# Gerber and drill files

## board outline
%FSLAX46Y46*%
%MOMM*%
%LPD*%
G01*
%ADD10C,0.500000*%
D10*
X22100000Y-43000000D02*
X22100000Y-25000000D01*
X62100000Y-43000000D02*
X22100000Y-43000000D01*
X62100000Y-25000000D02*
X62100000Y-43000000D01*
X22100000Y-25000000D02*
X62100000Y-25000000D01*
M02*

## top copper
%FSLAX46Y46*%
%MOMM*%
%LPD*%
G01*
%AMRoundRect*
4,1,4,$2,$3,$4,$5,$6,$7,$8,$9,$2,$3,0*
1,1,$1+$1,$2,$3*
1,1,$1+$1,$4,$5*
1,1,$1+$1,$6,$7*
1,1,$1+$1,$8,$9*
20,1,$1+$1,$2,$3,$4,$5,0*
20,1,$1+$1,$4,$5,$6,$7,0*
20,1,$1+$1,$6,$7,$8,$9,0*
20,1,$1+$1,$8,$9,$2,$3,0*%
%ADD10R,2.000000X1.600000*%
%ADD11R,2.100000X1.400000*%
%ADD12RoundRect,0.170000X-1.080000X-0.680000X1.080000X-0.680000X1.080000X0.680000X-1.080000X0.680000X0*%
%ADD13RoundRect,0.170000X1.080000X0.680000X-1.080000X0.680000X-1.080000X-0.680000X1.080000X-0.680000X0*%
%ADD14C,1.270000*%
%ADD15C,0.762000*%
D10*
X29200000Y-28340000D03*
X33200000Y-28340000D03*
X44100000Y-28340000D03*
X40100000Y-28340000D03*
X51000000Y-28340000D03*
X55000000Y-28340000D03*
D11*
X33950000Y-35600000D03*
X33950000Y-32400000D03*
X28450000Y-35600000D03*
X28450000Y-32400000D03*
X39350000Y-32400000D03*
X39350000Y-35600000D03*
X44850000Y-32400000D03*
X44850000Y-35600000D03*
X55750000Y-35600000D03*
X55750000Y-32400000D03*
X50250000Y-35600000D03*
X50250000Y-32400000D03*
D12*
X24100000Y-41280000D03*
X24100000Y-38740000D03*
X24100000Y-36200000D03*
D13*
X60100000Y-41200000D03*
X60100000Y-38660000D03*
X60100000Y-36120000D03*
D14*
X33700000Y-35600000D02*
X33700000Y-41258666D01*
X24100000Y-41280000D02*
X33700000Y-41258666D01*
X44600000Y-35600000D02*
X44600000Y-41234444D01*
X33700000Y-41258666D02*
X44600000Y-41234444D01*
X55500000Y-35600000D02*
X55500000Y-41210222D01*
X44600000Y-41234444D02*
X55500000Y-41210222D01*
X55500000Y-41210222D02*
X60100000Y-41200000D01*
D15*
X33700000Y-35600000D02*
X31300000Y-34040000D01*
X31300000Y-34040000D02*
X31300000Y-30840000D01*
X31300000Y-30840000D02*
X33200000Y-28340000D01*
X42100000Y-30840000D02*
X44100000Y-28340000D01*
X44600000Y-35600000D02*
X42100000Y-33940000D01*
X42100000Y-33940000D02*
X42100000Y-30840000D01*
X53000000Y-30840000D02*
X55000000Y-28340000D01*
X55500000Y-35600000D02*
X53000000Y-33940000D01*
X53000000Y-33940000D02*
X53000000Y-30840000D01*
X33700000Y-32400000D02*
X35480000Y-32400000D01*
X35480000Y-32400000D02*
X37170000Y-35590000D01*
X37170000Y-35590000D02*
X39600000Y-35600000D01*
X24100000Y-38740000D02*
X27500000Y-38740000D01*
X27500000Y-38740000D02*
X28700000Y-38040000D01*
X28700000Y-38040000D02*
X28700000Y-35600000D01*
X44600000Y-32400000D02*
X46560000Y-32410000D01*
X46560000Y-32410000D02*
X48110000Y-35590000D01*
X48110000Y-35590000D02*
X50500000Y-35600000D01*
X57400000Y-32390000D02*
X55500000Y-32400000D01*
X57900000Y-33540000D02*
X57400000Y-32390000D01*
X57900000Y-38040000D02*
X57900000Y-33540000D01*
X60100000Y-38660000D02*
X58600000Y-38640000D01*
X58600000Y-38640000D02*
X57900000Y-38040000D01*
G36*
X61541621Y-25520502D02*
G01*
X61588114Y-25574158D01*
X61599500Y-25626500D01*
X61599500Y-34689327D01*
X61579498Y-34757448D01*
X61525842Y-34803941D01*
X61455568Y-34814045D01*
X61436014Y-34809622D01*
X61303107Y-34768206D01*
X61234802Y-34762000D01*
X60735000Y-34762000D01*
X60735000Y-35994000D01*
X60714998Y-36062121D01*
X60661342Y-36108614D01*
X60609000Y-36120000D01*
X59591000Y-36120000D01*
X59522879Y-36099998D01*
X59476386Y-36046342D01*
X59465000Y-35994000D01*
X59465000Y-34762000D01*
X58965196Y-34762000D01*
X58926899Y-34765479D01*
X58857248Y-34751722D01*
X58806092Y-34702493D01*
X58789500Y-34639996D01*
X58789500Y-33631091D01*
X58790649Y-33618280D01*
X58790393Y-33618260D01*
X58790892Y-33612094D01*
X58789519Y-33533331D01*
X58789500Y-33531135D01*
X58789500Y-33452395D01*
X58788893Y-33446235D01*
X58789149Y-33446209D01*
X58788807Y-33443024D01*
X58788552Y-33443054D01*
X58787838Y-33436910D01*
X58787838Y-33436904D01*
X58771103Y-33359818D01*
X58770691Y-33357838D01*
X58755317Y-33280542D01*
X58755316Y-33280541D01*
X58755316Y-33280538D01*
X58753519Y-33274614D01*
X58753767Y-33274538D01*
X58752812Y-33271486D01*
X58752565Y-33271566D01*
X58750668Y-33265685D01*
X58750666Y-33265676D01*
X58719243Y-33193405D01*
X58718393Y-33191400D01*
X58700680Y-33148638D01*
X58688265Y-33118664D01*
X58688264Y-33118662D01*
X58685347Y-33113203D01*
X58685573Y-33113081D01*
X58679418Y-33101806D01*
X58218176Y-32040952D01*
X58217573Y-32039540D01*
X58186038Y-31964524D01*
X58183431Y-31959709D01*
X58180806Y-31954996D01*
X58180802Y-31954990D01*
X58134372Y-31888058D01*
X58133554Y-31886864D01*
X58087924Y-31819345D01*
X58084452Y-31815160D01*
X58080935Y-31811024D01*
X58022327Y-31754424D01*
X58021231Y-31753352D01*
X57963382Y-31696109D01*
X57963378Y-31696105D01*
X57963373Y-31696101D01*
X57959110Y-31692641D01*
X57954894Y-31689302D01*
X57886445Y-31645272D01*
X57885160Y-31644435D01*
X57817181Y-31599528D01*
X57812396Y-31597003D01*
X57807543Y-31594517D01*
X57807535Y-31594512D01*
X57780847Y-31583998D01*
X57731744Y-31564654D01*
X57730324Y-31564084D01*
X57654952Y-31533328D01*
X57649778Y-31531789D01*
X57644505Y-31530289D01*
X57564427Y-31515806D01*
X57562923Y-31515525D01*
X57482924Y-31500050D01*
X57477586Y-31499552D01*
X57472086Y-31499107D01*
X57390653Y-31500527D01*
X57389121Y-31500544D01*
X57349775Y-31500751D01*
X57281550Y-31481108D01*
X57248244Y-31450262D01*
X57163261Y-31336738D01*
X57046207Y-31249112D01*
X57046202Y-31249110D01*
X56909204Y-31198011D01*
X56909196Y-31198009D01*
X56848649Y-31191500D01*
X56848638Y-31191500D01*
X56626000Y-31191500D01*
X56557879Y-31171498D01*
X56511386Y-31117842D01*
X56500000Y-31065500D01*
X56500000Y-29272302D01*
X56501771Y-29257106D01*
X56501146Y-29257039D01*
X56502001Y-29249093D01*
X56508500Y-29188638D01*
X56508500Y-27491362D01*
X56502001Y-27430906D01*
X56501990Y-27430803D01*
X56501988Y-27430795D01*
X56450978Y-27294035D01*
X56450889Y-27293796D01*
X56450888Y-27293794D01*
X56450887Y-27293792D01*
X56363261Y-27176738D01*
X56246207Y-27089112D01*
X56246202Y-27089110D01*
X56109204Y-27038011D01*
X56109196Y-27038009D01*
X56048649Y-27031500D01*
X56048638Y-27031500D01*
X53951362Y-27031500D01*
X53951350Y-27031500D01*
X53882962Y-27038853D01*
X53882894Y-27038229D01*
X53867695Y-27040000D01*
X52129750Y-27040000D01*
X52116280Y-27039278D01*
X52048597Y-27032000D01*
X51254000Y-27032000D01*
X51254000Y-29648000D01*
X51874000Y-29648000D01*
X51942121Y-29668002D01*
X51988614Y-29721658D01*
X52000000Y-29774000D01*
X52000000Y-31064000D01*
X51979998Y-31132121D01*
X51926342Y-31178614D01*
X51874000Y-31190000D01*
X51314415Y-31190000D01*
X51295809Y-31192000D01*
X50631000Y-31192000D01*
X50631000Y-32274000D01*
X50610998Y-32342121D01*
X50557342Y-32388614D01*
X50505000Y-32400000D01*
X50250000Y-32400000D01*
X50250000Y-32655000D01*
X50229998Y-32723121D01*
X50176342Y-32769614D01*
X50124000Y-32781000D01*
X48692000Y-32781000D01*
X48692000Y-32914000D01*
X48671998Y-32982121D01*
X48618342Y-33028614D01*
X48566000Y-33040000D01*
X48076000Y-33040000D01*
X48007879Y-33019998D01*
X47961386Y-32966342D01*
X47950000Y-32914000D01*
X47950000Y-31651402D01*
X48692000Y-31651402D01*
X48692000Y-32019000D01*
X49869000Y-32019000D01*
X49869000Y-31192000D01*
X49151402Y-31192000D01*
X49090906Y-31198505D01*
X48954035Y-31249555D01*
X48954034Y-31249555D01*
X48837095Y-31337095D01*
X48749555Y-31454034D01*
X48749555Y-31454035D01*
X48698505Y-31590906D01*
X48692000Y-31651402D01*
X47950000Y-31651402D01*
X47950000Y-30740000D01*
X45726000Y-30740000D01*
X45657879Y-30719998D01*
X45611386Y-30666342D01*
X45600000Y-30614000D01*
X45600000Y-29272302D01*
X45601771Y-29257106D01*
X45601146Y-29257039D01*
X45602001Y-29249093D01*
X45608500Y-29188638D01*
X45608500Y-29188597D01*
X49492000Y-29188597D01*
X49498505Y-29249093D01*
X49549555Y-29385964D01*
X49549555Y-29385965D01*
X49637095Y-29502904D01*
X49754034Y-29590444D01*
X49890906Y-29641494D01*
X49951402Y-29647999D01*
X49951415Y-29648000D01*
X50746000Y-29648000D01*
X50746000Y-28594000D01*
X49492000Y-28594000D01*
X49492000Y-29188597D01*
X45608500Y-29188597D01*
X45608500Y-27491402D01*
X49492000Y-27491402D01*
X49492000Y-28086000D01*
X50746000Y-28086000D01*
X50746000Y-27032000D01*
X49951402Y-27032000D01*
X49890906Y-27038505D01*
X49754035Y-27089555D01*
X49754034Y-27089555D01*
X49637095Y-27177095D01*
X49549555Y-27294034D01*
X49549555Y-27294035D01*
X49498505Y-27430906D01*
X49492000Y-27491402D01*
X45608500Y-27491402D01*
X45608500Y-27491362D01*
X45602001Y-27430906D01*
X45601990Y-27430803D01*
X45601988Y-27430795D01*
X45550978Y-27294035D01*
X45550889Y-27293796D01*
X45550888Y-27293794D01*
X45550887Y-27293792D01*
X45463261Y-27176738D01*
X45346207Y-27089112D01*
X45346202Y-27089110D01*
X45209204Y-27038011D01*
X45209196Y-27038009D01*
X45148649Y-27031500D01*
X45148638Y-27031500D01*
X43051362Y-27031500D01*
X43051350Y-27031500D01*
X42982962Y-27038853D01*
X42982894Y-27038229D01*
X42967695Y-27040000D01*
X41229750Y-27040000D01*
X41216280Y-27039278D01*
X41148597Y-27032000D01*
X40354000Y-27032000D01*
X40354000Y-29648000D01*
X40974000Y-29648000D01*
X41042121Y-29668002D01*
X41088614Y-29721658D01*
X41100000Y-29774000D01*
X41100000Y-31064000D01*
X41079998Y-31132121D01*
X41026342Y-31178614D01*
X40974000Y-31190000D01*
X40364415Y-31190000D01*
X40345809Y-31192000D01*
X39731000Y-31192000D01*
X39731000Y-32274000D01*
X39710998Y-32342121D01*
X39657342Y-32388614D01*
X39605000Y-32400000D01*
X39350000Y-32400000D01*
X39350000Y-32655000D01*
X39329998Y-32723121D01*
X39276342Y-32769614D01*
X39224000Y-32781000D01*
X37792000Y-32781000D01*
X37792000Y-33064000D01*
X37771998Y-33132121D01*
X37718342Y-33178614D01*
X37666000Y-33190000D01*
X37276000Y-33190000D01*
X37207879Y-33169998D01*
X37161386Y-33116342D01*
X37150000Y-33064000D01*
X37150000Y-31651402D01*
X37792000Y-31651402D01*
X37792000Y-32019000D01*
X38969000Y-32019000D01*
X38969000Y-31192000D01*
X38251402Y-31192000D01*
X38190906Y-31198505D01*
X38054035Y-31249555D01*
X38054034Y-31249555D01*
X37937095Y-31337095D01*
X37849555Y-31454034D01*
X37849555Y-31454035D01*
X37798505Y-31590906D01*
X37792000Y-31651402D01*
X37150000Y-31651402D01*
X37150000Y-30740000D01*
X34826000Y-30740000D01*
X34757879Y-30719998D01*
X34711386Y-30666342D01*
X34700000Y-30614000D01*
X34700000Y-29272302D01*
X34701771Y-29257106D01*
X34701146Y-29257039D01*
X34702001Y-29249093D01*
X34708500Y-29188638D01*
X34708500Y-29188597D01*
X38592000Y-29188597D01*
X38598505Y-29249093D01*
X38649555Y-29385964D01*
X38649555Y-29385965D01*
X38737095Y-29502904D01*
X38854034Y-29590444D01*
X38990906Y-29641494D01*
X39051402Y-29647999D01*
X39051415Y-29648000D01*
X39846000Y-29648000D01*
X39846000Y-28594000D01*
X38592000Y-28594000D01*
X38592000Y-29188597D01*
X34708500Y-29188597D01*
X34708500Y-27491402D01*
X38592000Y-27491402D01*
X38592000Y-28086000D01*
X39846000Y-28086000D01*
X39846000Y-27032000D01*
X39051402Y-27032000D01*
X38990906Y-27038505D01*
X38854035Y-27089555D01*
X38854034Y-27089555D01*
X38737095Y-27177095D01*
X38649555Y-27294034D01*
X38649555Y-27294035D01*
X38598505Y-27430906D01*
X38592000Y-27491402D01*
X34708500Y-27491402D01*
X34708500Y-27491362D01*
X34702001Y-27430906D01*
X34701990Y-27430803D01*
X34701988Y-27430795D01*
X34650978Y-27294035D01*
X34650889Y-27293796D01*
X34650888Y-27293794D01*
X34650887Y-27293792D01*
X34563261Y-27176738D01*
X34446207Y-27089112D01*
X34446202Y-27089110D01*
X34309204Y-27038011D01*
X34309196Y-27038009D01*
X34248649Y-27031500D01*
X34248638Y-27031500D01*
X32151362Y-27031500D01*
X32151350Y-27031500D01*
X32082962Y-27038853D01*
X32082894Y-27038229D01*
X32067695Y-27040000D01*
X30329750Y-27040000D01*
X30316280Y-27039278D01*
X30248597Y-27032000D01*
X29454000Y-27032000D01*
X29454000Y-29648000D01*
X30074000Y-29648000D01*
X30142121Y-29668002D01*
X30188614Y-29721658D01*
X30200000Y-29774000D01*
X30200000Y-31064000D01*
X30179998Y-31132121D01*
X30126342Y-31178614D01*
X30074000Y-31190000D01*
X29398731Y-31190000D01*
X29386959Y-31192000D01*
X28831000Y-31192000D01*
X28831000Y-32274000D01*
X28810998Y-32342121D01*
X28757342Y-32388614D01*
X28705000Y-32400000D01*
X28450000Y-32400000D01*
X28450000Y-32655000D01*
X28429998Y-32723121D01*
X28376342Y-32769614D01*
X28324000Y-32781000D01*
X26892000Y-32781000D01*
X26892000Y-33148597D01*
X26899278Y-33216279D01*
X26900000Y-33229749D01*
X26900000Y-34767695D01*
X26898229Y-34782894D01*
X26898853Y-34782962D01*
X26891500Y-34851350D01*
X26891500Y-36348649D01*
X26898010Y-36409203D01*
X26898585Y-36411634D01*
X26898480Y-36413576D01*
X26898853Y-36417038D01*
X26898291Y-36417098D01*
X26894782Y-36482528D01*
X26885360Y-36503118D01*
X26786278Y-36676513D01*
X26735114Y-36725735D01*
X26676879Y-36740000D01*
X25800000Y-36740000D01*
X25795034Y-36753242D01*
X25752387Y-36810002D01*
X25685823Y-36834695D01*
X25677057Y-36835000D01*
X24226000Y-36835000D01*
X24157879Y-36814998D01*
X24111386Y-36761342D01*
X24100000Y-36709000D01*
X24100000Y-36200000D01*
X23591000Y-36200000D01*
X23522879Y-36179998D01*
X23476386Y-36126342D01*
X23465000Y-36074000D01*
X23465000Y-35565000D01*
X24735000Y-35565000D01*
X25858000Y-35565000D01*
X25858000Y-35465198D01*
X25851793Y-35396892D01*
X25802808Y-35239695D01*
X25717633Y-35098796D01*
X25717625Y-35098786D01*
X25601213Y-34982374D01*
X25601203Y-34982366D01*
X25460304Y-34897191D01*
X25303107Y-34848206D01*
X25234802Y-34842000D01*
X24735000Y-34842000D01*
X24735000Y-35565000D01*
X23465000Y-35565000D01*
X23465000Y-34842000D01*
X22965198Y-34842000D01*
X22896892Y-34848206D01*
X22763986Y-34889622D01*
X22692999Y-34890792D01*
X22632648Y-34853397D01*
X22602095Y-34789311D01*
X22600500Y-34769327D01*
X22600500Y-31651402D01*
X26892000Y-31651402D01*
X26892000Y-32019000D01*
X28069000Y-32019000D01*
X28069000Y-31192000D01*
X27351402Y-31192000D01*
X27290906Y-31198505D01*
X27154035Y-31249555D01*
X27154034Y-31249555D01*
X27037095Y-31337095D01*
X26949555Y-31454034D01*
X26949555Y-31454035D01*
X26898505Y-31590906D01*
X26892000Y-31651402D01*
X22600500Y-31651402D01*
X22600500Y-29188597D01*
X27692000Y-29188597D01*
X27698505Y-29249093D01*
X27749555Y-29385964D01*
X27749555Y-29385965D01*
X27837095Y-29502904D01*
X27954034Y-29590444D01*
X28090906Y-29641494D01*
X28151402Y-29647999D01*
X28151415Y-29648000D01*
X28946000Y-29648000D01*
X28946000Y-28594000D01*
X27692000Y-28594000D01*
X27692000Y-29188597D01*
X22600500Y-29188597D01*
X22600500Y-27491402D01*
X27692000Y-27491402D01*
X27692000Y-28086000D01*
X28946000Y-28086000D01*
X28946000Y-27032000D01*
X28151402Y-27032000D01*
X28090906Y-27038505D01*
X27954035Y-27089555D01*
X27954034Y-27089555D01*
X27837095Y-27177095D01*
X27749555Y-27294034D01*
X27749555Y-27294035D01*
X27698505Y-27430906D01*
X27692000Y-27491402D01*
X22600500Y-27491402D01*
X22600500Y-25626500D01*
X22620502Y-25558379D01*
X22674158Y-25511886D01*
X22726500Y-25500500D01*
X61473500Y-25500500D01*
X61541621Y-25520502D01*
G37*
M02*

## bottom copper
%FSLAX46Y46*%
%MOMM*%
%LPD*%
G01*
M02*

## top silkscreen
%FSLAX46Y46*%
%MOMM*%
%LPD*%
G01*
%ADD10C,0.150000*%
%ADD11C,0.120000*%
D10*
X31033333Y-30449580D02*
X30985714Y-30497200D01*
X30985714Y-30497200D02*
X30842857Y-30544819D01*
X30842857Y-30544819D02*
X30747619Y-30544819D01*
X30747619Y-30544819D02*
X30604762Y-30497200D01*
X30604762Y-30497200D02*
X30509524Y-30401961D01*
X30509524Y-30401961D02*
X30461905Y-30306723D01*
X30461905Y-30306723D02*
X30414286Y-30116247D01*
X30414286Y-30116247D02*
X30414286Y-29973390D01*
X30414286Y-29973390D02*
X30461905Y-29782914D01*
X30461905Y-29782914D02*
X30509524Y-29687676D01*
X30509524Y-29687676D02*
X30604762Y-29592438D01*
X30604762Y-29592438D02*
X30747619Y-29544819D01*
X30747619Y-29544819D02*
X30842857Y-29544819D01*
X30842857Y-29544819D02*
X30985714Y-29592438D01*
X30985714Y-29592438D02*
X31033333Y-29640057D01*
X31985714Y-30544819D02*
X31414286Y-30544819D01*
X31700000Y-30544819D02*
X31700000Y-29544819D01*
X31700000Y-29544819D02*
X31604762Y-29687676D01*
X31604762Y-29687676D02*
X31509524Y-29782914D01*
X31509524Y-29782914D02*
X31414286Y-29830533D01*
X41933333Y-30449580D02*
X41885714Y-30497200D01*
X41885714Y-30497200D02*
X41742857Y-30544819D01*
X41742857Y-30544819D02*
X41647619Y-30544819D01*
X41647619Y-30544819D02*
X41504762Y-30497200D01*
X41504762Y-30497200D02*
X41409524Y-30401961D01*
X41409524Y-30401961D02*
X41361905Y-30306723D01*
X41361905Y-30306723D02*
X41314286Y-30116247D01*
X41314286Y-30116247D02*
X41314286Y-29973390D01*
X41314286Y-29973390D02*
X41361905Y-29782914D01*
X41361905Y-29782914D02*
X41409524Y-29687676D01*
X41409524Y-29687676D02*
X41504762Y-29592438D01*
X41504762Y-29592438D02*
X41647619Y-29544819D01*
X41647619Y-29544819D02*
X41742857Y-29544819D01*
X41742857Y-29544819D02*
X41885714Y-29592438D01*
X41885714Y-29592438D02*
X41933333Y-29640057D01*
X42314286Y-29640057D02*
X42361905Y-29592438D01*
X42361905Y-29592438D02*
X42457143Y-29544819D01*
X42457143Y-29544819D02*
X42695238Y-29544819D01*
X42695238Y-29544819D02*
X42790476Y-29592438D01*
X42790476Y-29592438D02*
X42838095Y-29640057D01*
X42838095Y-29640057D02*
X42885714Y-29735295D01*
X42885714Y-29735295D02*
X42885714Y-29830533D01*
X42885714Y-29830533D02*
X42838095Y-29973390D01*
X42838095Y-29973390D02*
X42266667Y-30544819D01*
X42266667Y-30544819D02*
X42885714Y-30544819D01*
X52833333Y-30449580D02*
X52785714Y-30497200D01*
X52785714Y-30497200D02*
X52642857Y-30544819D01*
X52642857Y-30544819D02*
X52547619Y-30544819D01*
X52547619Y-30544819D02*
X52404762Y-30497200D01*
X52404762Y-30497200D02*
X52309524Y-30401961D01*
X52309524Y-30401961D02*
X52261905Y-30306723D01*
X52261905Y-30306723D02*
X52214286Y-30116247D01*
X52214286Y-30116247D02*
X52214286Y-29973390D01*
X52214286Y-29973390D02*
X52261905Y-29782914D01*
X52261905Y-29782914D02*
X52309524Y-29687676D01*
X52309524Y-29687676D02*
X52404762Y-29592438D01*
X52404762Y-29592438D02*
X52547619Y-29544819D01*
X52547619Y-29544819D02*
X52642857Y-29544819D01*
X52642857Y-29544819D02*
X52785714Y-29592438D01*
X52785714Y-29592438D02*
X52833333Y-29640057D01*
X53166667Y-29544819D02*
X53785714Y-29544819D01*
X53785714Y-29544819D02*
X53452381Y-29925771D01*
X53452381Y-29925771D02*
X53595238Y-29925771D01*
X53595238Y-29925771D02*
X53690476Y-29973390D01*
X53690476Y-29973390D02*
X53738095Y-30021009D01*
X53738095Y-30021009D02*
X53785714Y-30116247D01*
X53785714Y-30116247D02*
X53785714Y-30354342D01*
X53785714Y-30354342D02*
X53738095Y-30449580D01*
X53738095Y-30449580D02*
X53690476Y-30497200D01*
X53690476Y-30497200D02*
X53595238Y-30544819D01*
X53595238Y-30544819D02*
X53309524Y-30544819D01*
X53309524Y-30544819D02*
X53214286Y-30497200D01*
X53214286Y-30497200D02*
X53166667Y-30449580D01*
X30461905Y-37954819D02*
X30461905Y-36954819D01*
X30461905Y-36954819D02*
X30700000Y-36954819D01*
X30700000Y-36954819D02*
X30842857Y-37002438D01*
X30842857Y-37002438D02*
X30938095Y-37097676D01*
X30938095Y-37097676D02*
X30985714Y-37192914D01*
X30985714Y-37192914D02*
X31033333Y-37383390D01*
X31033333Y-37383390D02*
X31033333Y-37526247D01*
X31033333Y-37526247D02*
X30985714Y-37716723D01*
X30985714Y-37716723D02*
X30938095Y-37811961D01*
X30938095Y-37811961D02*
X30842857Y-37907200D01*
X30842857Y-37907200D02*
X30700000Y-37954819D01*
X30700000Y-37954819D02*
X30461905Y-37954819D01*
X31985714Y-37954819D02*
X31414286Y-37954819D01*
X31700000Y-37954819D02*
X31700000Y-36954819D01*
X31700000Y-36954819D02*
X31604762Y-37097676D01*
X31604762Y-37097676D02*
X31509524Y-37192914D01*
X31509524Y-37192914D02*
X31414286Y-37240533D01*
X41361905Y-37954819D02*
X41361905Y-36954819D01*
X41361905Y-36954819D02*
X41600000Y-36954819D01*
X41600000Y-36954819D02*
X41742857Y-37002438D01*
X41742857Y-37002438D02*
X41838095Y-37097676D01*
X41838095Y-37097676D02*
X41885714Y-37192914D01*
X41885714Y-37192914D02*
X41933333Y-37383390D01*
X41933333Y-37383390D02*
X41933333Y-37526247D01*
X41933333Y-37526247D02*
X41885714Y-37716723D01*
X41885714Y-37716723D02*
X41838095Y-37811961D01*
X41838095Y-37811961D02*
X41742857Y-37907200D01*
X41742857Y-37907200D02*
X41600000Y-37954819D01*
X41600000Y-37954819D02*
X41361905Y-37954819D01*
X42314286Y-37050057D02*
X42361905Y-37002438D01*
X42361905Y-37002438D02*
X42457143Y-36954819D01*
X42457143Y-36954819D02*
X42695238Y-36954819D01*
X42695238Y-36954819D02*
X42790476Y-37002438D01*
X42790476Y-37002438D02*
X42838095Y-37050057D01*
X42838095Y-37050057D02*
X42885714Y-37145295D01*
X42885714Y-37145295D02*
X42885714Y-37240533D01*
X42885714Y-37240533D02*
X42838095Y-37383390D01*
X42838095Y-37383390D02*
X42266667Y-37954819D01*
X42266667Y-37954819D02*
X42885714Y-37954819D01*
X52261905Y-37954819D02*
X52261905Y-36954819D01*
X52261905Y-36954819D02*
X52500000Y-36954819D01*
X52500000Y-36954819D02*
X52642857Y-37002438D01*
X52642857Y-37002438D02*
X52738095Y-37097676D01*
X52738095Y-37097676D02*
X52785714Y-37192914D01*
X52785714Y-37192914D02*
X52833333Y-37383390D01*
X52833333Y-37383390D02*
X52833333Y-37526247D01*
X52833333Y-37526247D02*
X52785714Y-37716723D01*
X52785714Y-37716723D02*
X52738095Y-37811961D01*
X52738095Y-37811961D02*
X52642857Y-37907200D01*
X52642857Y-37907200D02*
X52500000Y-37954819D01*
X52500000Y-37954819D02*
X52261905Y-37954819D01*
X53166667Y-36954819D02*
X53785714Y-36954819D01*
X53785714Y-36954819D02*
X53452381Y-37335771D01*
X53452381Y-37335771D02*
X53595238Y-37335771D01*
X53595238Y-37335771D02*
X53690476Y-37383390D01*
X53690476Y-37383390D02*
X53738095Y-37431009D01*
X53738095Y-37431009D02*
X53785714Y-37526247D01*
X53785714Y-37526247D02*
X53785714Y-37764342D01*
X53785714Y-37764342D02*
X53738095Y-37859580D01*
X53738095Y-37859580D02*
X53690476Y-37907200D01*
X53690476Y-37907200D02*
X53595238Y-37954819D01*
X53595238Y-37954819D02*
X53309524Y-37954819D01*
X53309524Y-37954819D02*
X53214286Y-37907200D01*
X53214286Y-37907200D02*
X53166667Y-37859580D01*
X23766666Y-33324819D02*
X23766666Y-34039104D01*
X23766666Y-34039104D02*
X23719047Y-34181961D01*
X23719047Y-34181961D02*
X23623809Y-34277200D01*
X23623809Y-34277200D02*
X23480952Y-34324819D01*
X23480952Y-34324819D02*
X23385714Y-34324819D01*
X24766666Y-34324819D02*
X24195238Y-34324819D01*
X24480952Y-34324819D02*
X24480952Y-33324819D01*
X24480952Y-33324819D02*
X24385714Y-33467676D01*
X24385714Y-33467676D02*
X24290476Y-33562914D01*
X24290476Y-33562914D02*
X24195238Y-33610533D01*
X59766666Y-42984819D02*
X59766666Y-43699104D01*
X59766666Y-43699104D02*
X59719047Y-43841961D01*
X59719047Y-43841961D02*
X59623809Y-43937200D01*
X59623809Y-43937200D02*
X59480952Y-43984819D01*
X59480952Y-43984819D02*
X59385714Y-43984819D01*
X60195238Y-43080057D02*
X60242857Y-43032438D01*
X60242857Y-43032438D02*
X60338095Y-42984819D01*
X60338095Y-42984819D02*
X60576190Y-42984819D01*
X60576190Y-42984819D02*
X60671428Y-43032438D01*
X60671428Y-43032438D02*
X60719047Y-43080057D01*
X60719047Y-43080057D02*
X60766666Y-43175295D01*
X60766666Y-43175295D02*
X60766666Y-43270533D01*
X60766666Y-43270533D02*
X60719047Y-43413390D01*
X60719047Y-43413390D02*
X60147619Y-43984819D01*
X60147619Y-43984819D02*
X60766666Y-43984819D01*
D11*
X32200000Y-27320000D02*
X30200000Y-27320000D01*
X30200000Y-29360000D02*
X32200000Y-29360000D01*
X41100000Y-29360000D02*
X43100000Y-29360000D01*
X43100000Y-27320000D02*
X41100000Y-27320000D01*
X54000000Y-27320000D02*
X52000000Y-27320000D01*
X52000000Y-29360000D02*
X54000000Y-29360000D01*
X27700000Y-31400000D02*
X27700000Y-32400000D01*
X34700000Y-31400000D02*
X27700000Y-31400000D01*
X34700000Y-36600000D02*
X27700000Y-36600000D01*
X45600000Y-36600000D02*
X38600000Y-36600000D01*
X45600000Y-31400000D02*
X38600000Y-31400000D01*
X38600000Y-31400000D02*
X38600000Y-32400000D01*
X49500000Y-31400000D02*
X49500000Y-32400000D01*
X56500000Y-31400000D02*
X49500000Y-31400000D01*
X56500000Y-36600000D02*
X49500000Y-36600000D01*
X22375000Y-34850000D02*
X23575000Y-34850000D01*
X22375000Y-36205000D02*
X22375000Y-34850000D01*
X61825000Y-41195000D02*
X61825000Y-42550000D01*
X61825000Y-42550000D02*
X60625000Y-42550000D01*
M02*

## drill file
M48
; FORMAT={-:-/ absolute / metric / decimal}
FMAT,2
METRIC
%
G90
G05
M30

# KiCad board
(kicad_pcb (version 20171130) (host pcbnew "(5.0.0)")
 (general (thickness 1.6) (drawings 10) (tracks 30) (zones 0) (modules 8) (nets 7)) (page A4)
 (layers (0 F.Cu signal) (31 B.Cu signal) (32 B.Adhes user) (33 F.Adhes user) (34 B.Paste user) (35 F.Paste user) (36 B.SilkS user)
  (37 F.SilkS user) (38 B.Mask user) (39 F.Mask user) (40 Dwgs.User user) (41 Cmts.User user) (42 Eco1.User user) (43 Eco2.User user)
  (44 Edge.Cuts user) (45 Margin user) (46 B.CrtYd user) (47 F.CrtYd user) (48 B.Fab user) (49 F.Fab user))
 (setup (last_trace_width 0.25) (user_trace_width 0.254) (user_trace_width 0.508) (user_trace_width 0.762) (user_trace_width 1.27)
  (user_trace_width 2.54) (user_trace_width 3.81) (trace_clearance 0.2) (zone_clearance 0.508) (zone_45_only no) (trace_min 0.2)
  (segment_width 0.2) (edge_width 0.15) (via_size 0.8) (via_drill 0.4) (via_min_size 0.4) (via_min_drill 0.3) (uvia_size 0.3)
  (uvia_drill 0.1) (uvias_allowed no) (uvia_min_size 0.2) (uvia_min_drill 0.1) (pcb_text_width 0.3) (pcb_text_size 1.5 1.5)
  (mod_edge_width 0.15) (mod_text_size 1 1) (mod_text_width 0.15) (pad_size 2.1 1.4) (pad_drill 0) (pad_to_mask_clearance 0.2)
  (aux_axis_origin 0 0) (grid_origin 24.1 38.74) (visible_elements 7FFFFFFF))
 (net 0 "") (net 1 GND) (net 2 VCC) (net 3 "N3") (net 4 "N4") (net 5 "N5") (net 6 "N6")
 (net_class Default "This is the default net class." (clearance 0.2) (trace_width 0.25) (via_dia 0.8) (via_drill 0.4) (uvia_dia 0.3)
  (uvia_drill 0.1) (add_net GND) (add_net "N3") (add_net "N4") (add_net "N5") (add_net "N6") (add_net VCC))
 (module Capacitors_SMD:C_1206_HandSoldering (layer F.Cu) (at 31.2 28.34 180)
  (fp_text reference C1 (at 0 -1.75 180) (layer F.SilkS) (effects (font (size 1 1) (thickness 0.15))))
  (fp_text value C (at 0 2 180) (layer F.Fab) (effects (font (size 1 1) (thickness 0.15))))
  (fp_line (start -1 1.02) (end 1 1.02) (layer F.SilkS) (width 0.12))
  (fp_line (start 1 -1.02) (end -1 -1.02) (layer F.SilkS) (width 0.12))
  (pad 2 smd rect (at 2 0 180) (size 2 1.6) (layers F.Cu F.Paste F.Mask) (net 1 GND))
  (pad 1 smd rect (at -2 0 180) (size 2 1.6) (layers F.Cu F.Paste F.Mask) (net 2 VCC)))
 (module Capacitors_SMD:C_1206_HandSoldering (layer F.Cu) (at 42.1 28.34 180)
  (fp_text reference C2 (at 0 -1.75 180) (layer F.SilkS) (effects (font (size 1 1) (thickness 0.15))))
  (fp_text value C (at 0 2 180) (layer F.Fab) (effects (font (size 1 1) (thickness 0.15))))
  (fp_line (start 1 -1.02) (end -1 -1.02) (layer F.SilkS) (width 0.12))
  (fp_line (start -1 1.02) (end 1 1.02) (layer F.SilkS) (width 0.12))
  (pad 1 smd rect (at -2 0 180) (size 2 1.6) (layers F.Cu F.Paste F.Mask) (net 2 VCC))
  (pad 2 smd rect (at 2 0 180) (size 2 1.6) (layers F.Cu F.Paste F.Mask) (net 1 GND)))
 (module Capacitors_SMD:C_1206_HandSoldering (layer F.Cu) (at 53 28.34 180)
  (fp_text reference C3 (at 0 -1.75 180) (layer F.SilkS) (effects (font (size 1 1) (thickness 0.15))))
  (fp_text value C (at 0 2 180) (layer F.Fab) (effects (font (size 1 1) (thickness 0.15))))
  (fp_line (start -1 1.02) (end 1 1.02) (layer F.SilkS) (width 0.12))
  (fp_line (start 1 -1.02) (end -1 -1.02) (layer F.SilkS) (width 0.12))
  (pad 2 smd rect (at 2 0 180) (size 2 1.6) (layers F.Cu F.Paste F.Mask) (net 1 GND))
  (pad 1 smd rect (at -2 0 180) (size 2 1.6) (layers F.Cu F.Paste F.Mask) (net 2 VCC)))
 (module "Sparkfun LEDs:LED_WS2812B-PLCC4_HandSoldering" (layer F.Cu) (at 31.2 34 180)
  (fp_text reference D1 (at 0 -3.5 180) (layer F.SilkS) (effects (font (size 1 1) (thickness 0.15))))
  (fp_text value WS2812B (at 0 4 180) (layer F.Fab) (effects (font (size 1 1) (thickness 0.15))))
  (fp_line (start 3.5 2.6) (end 3.5 1.6) (layer F.SilkS) (width 0.12))
  (fp_line (start -3.5 2.6) (end 3.5 2.6) (layer F.SilkS) (width 0.12))
  (fp_line (start -3.5 -2.6) (end 3.5 -2.6) (layer F.SilkS) (width 0.12))
  (pad 1 smd rect (at -2.5 -1.6 180) (size 2.1 1.4) (drill (offset -0.25 0)) (layers F.Cu F.Paste F.Mask) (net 2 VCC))
  (pad 2 smd rect (at -2.5 1.6 180) (size 2.1 1.4) (drill (offset -0.25 0)) (layers F.Cu F.Paste F.Mask) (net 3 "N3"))
  (pad 4 smd rect (at 2.5 -1.6 180) (size 2.1 1.4) (drill (offset 0.25 0)) (layers F.Cu F.Paste F.Mask) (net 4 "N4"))
  (pad 3 smd rect (at 2.5 1.6 180) (size 2.1 1.4) (drill (offset 0.25 0)) (layers F.Cu F.Paste F.Mask) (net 1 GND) (thermal_width 0.762)))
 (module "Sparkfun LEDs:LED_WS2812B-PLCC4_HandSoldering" (layer F.Cu) (at 42.1 34 180)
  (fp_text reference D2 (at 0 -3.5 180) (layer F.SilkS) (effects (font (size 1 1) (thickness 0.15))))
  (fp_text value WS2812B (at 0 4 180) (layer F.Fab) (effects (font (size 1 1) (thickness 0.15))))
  (fp_line (start -3.5 -2.6) (end 3.5 -2.6) (layer F.SilkS) (width 0.12))
  (fp_line (start -3.5 2.6) (end 3.5 2.6) (layer F.SilkS) (width 0.12))
  (fp_line (start 3.5 2.6) (end 3.5 1.6) (layer F.SilkS) (width 0.12))
  (pad 3 smd rect (at 2.5 1.6 180) (size 2.1 1.4) (drill (offset 0.25 0)) (layers F.Cu F.Paste F.Mask) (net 1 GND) (thermal_width 0.762))
  (pad 4 smd rect (at 2.5 -1.6 180) (size 2.1 1.4) (drill (offset 0.25 0)) (layers F.Cu F.Paste F.Mask) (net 3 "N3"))
  (pad 2 smd rect (at -2.5 1.6 180) (size 2.1 1.4) (drill (offset -0.25 0)) (layers F.Cu F.Paste F.Mask) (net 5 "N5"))
  (pad 1 smd rect (at -2.5 -1.6 180) (size 2.1 1.4) (drill (offset -0.25 0)) (layers F.Cu F.Paste F.Mask) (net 2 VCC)))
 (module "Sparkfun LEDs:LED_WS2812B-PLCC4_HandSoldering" (layer F.Cu) (at 53 34 180)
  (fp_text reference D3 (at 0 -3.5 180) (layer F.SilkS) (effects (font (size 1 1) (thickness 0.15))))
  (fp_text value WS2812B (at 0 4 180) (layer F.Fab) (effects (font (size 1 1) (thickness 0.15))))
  (fp_line (start 3.5 2.6) (end 3.5 1.6) (layer F.SilkS) (width 0.12))
  (fp_line (start -3.5 2.6) (end 3.5 2.6) (layer F.SilkS) (width 0.12))
  (fp_line (start -3.5 -2.6) (end 3.5 -2.6) (layer F.SilkS) (width 0.12))
  (pad 1 smd rect (at -2.5 -1.6 180) (size 2.1 1.4) (drill (offset -0.25 0)) (layers F.Cu F.Paste F.Mask) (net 2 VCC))
  (pad 2 smd rect (at -2.5 1.6 180) (size 2.1 1.4) (drill (offset -0.25 0)) (layers F.Cu F.Paste F.Mask) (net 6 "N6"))
  (pad 4 smd rect (at 2.5 -1.6 180) (size 2.1 1.4) (drill (offset 0.25 0)) (layers F.Cu F.Paste F.Mask) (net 5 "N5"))
  (pad 3 smd rect (at 2.5 1.6 180) (size 2.1 1.4) (drill (offset 0.25 0)) (layers F.Cu F.Paste F.Mask) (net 1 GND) (thermal_width 0.762)))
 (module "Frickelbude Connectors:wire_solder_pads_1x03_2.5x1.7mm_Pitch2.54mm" (layer F.Cu) (at 24.1 36.2)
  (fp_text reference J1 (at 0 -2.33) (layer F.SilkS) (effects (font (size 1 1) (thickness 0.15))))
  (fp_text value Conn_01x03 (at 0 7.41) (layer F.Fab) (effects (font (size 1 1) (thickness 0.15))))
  (fp_line (start -1.725 -1.35) (end -0.525 -1.35) (layer F.SilkS) (width 0.12))
  (fp_line (start -1.725 0.005) (end -1.725 -1.35) (layer F.SilkS) (width 0.12))
  (pad 3 connect roundrect (at 0 5.08) (size 2.5 1.7) (layers F.Cu F.Mask) (roundrect_rratio 0.1) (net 2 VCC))
  (pad 2 connect roundrect (at 0 2.54) (size 2.5 1.7) (layers F.Cu F.Mask) (roundrect_rratio 0.1) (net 4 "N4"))
  (pad 1 connect roundrect (at 0 0) (size 2.5 1.7) (layers F.Cu F.Mask) (roundrect_rratio 0.1) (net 1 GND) (thermal_width 1.27)))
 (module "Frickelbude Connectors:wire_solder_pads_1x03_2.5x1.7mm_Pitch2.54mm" (layer F.Cu) (at 60.1 41.2 180)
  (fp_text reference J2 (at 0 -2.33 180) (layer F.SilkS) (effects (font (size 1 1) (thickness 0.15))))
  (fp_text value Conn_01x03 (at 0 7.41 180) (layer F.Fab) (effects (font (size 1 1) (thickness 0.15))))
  (fp_line (start -1.725 0.005) (end -1.725 -1.35) (layer F.SilkS) (width 0.12))
  (fp_line (start -1.725 -1.35) (end -0.525 -1.35) (layer F.SilkS) (width 0.12))
  (pad 1 connect roundrect (at 0 0 180) (size 2.5 1.7) (layers F.Cu F.Mask) (roundrect_rratio 0.1) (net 2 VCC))
  (pad 2 connect roundrect (at 0 2.54 180) (size 2.5 1.7) (layers F.Cu F.Mask) (roundrect_rratio 0.1) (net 6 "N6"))
  (pad 3 connect roundrect (at 0 5.08 180) (size 2.5 1.7) (layers F.Cu F.Mask) (roundrect_rratio 0.1) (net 1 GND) (zone_connect 1)
   (thermal_width 1.27)))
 (gr_line (start 22.1 43) (end 22.1 25) (layer Edge.Cuts) (width 0.5))
 (gr_line (start 62.1 43) (end 22.1 43) (layer Edge.Cuts) (width 0.5))
 (gr_line (start 62.1 25) (end 62.1 43) (layer Edge.Cuts) (width 0.5))
 (gr_line (start 22.1 25) (end 62.1 25) (layer Edge.Cuts) (width 0.5))
 (segment (start 33.7 35.6) (end 33.7 41.258666) (width 1.27) (layer F.Cu) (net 2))
 (segment (start 24.1 41.28) (end 33.7 41.258666) (width 1.27) (layer F.Cu) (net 2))
 (segment (start 44.6 35.6) (end 44.6 41.234444) (width 1.27) (layer F.Cu) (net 2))
 (segment (start 33.7 41.258666) (end 44.6 41.234444) (width 1.27) (layer F.Cu) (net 2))
 (segment (start 55.5 35.6) (end 55.5 41.210222) (width 1.27) (layer F.Cu) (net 2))
 (segment (start 44.6 41.234444) (end 55.5 41.210222) (width 1.27) (layer F.Cu) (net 2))
 (segment (start 55.5 41.210222) (end 60.1 41.2) (width 1.27) (layer F.Cu) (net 2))
 (segment (start 33.7 35.6) (end 31.3 34.04) (width 0.762) (layer F.Cu) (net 2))
 (segment (start 31.3 34.04) (end 31.3 30.84) (width 0.762) (layer F.Cu) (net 2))
 (segment (start 31.3 30.84) (end 33.2 28.34) (width 0.762) (layer F.Cu) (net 2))
 (segment (start 42.1 30.84) (end 44.1 28.34) (width 0.762) (layer F.Cu) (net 2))
 (segment (start 44.6 35.6) (end 42.1 33.94) (width 0.762) (layer F.Cu) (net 2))
 (segment (start 42.1 33.94) (end 42.1 30.84) (width 0.762) (layer F.Cu) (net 2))
 (segment (start 53 30.84) (end 55 28.34) (width 0.762) (layer F.Cu) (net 2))
 (segment (start 55.5 35.6) (end 53 33.94) (width 0.762) (layer F.Cu) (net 2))
 (segment (start 53 33.94) (end 53 30.84) (width 0.762) (layer F.Cu) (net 2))
 (segment (start 33.7 32.4) (end 35.48 32.4) (width 0.762) (layer F.Cu) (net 3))
 (segment (start 35.48 32.4) (end 37.17 35.59) (width 0.762) (layer F.Cu) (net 3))
 (segment (start 37.17 35.59) (end 39.6 35.6) (width 0.762) (layer F.Cu) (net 3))
 (segment (start 24.1 38.74) (end 27.5 38.74) (width 0.762) (layer F.Cu) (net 4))
 (segment (start 27.5 38.74) (end 28.7 38.04) (width 0.762) (layer F.Cu) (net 4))
 (segment (start 28.7 38.04) (end 28.7 35.6) (width 0.762) (layer F.Cu) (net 4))
 (segment (start 44.6 32.4) (end 46.56 32.41) (width 0.762) (layer F.Cu) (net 5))
 (segment (start 46.56 32.41) (end 48.11 35.59) (width 0.762) (layer F.Cu) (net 5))
 (segment (start 48.11 35.59) (end 50.5 35.6) (width 0.762) (layer F.Cu) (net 5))
 (segment (start 57.4 32.39) (end 55.5 32.4) (width 0.762) (layer F.Cu) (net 6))
 (segment (start 57.9 33.54) (end 57.4 32.39) (width 0.762) (layer F.Cu) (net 6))
 (segment (start 57.9 38.04) (end 57.9 33.54) (width 0.762) (layer F.Cu) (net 6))
 (segment (start 60.1 38.66) (end 58.6 38.64) (width 0.762) (layer F.Cu) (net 6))
 (segment (start 58.6 38.64) (end 57.9 38.04) (width 0.762) (layer F.Cu) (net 6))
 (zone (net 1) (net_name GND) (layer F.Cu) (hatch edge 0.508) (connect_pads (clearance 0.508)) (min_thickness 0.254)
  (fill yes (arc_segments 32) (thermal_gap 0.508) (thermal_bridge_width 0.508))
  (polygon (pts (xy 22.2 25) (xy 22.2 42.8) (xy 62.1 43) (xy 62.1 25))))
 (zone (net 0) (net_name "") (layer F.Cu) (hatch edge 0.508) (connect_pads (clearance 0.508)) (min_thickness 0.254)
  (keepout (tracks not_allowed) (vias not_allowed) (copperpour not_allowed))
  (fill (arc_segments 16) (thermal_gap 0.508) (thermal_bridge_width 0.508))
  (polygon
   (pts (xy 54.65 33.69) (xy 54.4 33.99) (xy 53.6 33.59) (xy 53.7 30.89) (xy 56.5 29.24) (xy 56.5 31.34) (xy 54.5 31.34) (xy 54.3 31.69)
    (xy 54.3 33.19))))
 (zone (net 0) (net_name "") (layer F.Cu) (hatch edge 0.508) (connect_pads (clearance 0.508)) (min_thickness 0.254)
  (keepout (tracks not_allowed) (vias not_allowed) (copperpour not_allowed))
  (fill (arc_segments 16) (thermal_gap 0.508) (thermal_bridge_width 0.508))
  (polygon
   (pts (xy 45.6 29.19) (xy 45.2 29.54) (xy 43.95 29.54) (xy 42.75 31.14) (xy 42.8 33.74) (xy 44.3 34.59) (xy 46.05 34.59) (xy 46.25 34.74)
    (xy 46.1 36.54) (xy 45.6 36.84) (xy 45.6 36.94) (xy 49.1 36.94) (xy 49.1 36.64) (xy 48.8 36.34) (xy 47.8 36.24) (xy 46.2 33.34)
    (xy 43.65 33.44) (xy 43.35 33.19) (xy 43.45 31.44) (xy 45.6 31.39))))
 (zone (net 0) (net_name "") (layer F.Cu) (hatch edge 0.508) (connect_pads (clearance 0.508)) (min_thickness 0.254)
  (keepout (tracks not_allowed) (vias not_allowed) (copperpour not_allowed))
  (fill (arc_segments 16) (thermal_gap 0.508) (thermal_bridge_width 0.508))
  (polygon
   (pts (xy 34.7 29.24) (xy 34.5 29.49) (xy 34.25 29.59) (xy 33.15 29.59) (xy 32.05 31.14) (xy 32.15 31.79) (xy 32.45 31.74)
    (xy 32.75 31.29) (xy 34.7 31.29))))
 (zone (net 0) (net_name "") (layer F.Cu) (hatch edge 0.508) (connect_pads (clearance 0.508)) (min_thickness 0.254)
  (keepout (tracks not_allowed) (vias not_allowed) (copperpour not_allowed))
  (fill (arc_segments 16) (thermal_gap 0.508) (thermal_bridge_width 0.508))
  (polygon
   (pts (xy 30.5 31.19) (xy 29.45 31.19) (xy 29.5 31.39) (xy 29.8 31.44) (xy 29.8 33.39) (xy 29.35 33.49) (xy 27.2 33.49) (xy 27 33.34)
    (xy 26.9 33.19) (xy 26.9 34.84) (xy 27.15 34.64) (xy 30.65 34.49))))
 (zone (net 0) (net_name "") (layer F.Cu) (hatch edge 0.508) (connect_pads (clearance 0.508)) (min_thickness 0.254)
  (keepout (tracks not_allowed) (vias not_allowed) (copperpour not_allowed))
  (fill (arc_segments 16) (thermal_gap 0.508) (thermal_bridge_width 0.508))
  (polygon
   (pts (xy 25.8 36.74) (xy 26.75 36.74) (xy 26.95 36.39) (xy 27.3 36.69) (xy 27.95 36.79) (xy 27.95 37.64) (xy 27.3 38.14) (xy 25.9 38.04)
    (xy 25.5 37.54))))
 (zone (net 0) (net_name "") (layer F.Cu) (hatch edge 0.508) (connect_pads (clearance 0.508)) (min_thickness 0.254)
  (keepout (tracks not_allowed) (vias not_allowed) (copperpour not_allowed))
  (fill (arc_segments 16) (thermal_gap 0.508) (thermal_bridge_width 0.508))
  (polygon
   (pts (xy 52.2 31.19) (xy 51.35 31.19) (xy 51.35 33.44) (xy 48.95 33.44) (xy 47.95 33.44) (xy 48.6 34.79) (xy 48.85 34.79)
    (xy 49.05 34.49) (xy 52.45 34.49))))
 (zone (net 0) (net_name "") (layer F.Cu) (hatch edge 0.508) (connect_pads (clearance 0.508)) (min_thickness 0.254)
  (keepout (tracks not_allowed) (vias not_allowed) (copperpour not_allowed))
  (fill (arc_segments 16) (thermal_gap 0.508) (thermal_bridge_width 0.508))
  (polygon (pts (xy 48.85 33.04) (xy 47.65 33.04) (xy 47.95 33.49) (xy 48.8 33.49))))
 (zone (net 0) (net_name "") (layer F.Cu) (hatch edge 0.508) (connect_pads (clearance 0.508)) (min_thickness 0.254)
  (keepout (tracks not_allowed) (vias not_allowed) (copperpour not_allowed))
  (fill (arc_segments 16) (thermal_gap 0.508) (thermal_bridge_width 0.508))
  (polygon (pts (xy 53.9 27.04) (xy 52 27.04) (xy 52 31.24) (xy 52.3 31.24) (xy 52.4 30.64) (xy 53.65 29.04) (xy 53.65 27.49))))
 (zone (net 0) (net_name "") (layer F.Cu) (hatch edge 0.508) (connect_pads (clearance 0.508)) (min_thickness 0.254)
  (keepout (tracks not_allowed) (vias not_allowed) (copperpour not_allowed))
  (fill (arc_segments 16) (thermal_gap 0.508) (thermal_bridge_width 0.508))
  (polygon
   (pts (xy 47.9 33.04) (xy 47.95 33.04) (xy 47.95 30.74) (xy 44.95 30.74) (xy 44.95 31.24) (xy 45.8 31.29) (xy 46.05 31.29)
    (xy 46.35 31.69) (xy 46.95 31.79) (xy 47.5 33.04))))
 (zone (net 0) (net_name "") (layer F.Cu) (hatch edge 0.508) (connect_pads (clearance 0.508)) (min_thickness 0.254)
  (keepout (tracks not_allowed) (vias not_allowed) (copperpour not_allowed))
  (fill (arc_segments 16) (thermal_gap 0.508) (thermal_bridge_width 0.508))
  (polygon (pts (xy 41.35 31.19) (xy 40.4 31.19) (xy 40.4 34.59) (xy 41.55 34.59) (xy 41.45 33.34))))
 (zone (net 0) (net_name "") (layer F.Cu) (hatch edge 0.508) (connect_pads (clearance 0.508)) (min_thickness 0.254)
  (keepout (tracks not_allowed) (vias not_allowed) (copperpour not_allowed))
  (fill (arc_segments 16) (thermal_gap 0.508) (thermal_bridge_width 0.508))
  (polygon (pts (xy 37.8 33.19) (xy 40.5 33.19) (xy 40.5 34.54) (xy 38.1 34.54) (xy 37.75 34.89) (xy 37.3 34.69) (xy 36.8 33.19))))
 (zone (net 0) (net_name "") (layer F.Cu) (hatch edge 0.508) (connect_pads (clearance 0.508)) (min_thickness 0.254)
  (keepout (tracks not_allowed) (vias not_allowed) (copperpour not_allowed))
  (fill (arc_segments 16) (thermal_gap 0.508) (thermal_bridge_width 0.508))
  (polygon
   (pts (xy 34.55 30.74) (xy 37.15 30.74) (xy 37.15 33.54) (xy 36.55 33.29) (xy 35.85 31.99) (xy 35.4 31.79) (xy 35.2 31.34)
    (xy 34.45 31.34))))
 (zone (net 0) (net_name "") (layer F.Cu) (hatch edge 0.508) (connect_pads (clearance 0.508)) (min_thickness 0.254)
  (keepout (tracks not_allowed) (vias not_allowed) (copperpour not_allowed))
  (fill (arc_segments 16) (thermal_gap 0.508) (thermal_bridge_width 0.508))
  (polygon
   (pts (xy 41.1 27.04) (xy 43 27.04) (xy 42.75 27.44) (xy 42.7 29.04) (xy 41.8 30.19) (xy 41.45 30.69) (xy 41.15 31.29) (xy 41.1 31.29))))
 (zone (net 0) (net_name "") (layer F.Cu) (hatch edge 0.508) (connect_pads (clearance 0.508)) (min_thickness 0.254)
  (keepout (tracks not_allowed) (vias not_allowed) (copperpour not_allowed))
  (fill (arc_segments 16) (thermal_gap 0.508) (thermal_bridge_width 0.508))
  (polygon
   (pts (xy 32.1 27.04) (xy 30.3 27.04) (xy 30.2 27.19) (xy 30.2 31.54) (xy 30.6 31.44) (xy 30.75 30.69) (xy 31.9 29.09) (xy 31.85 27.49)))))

